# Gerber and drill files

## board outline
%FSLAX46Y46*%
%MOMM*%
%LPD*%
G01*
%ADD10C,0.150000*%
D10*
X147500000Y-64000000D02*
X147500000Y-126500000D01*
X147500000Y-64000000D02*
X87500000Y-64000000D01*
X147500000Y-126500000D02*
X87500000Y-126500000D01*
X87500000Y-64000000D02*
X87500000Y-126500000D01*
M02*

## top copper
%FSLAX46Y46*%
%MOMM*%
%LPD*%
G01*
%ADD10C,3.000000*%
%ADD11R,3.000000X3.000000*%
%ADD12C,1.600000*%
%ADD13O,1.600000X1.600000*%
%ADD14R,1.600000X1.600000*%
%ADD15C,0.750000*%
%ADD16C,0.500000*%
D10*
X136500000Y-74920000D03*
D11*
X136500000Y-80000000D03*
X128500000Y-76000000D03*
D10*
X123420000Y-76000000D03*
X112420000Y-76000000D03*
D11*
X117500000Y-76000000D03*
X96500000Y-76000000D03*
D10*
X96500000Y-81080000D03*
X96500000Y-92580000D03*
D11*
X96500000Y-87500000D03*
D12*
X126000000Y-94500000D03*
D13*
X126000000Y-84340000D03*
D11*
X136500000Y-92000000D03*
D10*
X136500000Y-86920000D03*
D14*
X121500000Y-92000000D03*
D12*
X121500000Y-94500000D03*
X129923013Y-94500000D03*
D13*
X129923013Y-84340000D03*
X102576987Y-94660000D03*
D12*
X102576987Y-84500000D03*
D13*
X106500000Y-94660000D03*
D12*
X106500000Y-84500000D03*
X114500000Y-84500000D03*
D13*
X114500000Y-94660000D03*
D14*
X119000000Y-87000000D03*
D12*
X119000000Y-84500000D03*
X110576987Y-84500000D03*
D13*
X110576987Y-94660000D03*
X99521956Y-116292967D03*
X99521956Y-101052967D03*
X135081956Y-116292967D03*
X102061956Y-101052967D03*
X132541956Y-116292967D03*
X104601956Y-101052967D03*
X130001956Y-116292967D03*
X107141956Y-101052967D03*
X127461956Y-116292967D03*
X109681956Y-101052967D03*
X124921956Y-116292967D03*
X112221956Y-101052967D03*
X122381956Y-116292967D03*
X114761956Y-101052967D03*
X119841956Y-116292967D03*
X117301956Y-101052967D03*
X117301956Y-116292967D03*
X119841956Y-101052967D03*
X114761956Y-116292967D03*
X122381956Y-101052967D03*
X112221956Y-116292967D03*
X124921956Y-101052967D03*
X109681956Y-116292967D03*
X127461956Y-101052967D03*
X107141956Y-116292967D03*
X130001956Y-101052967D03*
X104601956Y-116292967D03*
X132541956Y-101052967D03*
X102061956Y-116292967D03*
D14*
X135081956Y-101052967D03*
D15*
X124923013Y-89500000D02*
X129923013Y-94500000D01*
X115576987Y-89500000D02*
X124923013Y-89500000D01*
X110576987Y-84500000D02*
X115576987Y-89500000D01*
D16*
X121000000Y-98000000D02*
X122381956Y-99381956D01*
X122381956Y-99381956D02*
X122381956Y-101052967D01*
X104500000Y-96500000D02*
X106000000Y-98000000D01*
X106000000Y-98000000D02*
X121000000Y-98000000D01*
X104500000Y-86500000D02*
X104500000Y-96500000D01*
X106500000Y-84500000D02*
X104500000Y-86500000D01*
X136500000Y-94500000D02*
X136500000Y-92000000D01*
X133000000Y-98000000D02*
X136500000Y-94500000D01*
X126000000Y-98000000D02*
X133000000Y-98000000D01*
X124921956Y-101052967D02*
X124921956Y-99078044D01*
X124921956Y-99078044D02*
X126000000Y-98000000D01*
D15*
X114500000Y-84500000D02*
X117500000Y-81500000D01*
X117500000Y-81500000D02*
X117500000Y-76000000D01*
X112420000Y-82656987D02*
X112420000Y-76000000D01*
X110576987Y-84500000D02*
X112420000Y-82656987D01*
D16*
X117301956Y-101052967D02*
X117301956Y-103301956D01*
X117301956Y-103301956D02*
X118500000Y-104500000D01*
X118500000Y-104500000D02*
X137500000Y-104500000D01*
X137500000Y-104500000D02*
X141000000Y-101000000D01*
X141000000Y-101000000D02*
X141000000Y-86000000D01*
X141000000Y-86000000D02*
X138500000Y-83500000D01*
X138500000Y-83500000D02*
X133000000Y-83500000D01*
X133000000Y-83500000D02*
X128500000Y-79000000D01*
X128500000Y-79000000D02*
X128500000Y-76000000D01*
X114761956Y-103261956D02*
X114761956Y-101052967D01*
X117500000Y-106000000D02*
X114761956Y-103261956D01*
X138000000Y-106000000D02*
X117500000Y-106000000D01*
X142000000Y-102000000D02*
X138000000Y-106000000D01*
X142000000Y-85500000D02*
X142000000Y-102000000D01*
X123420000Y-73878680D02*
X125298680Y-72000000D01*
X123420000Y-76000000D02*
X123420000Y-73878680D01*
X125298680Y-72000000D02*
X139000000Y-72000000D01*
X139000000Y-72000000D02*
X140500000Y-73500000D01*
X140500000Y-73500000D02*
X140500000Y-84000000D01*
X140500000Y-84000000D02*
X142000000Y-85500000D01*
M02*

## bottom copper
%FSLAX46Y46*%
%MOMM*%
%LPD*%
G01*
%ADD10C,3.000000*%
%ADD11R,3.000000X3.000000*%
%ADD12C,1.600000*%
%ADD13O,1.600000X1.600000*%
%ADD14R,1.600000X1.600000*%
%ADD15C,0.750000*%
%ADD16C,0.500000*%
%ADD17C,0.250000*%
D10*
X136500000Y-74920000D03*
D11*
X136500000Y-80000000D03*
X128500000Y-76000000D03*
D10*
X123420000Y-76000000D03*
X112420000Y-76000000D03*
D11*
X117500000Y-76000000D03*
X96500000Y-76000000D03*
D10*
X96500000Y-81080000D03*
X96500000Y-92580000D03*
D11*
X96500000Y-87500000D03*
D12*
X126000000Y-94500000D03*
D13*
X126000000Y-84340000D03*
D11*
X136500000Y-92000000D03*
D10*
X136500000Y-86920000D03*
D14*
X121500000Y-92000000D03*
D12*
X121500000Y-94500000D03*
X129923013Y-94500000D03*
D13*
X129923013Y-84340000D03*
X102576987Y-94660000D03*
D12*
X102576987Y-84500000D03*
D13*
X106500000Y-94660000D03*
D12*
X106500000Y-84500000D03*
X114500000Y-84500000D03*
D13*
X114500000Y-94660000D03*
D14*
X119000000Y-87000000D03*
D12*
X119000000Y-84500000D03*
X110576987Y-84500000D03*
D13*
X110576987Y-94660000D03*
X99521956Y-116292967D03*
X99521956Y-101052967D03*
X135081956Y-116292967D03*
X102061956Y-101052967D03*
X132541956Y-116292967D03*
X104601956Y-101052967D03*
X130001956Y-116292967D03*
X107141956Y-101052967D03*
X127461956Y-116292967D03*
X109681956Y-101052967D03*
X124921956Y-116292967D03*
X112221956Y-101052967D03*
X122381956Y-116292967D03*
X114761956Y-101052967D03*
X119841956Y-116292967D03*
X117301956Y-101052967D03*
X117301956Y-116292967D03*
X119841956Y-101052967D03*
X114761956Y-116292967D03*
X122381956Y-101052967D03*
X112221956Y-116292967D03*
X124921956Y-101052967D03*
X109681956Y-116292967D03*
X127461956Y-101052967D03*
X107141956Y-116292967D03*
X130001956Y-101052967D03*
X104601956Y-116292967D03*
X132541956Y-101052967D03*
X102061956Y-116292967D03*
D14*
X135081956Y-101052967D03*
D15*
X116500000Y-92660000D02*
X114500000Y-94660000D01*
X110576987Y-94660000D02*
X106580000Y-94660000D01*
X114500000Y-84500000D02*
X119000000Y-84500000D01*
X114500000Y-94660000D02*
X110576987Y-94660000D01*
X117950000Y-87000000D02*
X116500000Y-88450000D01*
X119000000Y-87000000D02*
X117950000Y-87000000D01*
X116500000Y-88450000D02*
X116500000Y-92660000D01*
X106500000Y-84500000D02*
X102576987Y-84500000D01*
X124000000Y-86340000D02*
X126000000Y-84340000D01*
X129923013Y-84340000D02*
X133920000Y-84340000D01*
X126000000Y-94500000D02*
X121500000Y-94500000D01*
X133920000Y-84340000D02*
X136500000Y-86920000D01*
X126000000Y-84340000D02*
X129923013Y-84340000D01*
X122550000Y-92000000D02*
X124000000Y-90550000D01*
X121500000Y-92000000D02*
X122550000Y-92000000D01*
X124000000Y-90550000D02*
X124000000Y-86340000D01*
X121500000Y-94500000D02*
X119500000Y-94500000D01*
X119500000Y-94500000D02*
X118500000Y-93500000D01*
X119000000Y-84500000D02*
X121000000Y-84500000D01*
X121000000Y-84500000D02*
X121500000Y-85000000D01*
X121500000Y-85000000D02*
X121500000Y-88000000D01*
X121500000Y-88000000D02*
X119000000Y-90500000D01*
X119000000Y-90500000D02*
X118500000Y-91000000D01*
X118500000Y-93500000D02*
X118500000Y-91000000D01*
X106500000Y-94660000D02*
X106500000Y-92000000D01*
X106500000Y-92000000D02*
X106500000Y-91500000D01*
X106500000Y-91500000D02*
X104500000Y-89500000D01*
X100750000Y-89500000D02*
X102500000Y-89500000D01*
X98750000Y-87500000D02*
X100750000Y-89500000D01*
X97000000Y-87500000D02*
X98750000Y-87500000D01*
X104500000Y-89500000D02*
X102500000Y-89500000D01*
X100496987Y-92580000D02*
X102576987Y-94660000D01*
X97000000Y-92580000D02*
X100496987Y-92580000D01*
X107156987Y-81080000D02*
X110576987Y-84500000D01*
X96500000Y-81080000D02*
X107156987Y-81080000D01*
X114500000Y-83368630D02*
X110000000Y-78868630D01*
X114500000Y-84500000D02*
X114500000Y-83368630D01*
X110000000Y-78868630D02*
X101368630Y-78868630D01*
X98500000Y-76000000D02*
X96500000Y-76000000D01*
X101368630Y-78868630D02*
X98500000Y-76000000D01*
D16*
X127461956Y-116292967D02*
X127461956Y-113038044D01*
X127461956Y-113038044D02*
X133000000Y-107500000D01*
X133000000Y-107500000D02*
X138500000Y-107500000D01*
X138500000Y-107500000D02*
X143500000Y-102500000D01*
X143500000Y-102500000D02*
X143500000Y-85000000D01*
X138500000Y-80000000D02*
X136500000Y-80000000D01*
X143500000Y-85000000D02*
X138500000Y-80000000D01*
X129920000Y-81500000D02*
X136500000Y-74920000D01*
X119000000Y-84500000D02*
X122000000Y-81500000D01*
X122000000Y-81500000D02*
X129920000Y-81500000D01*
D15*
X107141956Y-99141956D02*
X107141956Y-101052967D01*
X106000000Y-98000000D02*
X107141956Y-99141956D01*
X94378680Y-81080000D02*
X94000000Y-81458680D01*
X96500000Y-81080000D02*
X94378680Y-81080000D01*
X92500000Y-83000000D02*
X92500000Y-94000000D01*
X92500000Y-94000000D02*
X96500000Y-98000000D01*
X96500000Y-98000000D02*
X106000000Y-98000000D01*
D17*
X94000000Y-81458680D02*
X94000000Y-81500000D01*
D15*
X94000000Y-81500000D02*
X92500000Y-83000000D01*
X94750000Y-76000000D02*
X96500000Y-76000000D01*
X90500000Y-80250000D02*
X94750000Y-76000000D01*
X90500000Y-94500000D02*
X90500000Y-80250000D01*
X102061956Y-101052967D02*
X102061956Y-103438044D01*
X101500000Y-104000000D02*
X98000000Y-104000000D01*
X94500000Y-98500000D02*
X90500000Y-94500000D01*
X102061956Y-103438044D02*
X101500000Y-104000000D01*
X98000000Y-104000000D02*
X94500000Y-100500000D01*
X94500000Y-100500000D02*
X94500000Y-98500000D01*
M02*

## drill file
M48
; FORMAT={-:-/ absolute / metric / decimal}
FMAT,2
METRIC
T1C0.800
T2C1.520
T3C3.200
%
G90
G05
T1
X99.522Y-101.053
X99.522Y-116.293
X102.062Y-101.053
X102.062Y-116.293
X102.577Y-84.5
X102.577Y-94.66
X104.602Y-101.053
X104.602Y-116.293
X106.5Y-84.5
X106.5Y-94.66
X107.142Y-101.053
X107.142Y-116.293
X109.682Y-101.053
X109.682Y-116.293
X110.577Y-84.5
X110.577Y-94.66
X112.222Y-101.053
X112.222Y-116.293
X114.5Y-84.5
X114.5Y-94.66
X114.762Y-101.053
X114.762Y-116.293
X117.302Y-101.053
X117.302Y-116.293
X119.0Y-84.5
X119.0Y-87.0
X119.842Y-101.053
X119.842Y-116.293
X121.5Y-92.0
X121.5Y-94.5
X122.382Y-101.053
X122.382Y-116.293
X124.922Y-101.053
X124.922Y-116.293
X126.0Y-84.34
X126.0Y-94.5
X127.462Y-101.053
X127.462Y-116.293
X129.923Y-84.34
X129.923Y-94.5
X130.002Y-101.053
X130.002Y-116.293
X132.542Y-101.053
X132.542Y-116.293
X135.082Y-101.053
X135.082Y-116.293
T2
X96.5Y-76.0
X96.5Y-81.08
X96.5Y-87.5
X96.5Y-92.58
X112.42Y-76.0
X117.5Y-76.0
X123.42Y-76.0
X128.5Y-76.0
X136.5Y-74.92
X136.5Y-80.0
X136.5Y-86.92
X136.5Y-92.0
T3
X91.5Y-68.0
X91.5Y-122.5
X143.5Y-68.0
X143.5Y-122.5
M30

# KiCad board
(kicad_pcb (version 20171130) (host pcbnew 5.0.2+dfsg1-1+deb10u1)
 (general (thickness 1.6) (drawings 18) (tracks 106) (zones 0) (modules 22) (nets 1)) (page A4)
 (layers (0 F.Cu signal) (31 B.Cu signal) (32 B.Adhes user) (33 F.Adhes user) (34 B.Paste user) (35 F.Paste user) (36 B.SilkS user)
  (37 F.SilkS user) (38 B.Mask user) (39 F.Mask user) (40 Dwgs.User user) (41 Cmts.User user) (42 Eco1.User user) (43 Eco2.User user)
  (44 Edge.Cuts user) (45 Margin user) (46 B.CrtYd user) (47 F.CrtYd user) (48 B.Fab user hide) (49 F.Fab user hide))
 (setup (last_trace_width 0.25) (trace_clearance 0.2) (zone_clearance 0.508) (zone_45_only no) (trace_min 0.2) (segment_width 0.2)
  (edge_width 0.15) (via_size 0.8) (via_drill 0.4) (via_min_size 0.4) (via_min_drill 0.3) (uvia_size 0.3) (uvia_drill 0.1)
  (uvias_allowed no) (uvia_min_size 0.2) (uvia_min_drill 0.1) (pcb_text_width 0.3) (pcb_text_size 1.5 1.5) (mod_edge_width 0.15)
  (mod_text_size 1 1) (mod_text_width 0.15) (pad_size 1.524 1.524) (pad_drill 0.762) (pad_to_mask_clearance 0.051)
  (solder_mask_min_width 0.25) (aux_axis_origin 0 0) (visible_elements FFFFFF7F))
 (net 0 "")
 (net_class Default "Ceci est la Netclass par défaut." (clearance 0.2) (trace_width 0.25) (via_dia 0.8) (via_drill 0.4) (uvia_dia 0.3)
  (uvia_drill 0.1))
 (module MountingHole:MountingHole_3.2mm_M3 (layer F.Cu) (at 91.5 68)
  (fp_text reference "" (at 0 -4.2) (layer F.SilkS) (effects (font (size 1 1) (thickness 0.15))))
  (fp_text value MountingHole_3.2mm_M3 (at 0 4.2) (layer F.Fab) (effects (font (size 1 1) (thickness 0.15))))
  (pad 1 np_thru_hole circle (at 0 0) (size 3.2 3.2) (drill 3.2) (layers *.Cu *.Mask)))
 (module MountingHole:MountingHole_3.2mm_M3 (layer F.Cu) (at 143.5 68)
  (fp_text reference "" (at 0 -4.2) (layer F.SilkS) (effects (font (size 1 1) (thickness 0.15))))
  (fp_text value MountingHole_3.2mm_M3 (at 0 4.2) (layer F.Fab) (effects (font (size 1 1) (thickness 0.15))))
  (pad 1 np_thru_hole circle (at 0 0) (size 3.2 3.2) (drill 3.2) (layers *.Cu *.Mask)))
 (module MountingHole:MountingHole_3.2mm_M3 (layer F.Cu) (at 143.5 122.5)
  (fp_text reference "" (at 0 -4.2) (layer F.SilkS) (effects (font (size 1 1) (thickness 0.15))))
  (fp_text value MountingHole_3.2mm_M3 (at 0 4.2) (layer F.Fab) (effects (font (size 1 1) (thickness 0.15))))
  (pad 1 np_thru_hole circle (at 0 0) (size 3.2 3.2) (drill 3.2) (layers *.Cu *.Mask)))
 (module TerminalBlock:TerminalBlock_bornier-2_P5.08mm (layer F.Cu) (at 136.5 80 90)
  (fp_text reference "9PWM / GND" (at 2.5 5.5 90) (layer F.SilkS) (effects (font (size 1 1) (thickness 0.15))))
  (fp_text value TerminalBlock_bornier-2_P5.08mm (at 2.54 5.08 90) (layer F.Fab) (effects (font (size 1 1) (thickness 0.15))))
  (pad 2 thru_hole circle (at 5.08 0 90) (size 3 3) (drill 1.52) (layers *.Cu *.Mask))
  (pad 1 thru_hole rect (at 0 0 90) (size 3 3) (drill 1.52) (layers *.Cu *.Mask)))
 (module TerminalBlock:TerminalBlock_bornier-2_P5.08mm (layer F.Cu) (at 128.5 76 180)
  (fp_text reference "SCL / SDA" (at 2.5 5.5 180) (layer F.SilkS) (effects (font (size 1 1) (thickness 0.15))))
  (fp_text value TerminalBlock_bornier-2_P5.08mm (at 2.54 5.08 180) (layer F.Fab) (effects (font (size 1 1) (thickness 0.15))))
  (pad 1 thru_hole rect (at 0 0 180) (size 3 3) (drill 1.52) (layers *.Cu *.Mask))
  (pad 2 thru_hole circle (at 5.08 0 180) (size 3 3) (drill 1.52) (layers *.Cu *.Mask)))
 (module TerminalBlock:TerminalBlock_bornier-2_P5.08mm (layer F.Cu) (at 117.5 76 180)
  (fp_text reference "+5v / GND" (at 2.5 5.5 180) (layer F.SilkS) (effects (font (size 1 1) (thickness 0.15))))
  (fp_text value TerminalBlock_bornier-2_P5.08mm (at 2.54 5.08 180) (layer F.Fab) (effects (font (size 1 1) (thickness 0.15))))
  (pad 2 thru_hole circle (at 5.08 0 180) (size 3 3) (drill 1.52) (layers *.Cu *.Mask))
  (pad 1 thru_hole rect (at 0 0 180) (size 3 3) (drill 1.52) (layers *.Cu *.Mask)))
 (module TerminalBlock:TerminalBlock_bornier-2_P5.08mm (layer F.Cu) (at 96.5 76 270)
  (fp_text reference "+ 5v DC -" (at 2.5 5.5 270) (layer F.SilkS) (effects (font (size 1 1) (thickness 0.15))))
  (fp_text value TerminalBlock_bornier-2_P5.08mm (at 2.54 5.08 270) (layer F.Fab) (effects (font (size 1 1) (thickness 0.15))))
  (pad 1 thru_hole rect (at 0 0 270) (size 3 3) (drill 1.52) (layers *.Cu *.Mask))
  (pad 2 thru_hole circle (at 5.08 0 270) (size 3 3) (drill 1.52) (layers *.Cu *.Mask)))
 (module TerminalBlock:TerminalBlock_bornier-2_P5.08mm (layer F.Cu) (at 96.5 87.5 270)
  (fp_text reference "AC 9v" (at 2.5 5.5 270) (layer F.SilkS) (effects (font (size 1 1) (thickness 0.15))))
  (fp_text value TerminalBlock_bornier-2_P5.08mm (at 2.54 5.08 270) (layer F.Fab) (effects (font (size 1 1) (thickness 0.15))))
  (pad 2 thru_hole circle (at 5.08 0 270) (size 3 3) (drill 1.52) (layers *.Cu *.Mask))
  (pad 1 thru_hole rect (at 0 0 270) (size 3 3) (drill 1.52) (layers *.Cu *.Mask)))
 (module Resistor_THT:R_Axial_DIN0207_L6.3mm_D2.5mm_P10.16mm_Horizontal (layer F.Cu) (at 126 94.5 90)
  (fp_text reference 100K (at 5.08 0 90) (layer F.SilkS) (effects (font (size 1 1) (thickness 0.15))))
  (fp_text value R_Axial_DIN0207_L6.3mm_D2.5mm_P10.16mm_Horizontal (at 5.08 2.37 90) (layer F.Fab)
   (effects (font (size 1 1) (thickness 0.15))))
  (pad 1 thru_hole circle (at 0 0 90) (size 1.6 1.6) (drill 0.8) (layers *.Cu *.Mask))
  (pad 2 thru_hole oval (at 10.16 0 90) (size 1.6 1.6) (drill 0.8) (layers *.Cu *.Mask)))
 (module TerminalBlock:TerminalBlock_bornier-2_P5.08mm (layer F.Cu) (at 136.5 92 90)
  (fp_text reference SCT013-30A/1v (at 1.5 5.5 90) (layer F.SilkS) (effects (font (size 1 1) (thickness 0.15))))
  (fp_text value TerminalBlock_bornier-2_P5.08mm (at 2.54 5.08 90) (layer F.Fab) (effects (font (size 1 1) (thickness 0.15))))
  (pad 1 thru_hole rect (at 0 0 90) (size 3 3) (drill 1.52) (layers *.Cu *.Mask))
  (pad 2 thru_hole circle (at 5.08 0 90) (size 3 3) (drill 1.52) (layers *.Cu *.Mask)))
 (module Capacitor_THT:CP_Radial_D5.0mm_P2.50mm (layer F.Cu) (at 121.5 92 270)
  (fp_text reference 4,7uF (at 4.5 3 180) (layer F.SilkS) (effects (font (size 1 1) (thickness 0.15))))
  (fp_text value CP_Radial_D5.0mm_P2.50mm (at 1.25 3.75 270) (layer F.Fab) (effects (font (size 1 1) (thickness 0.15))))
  (pad 1 thru_hole rect (at 0 0 270) (size 1.6 1.6) (drill 0.8) (layers *.Cu *.Mask))
  (pad 2 thru_hole circle (at 2.5 0 270) (size 1.6 1.6) (drill 0.8) (layers *.Cu *.Mask)))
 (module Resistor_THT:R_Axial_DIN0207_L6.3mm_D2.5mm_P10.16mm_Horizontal (layer F.Cu) (at 129.923013 94.5 90)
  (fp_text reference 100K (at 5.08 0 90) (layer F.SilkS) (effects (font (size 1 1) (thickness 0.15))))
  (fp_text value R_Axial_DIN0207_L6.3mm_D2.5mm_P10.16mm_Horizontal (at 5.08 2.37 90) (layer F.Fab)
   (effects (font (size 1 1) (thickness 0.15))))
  (pad 1 thru_hole circle (at 0 0 90) (size 1.6 1.6) (drill 0.8) (layers *.Cu *.Mask))
  (pad 2 thru_hole oval (at 10.16 0 90) (size 1.6 1.6) (drill 0.8) (layers *.Cu *.Mask)))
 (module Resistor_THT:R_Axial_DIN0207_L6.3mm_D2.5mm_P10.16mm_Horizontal (layer F.Cu) (at 102.576987 84.5 270)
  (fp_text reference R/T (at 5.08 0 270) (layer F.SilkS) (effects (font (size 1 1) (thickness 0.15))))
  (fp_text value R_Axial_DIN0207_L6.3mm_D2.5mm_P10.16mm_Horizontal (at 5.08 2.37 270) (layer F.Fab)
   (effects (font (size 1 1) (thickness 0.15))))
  (pad 2 thru_hole oval (at 10.16 0 270) (size 1.6 1.6) (drill 0.8) (layers *.Cu *.Mask))
  (pad 1 thru_hole circle (at 0 0 270) (size 1.6 1.6) (drill 0.8) (layers *.Cu *.Mask)))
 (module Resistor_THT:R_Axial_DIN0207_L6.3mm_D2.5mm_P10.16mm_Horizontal (layer F.Cu) (at 106.5 84.5 270)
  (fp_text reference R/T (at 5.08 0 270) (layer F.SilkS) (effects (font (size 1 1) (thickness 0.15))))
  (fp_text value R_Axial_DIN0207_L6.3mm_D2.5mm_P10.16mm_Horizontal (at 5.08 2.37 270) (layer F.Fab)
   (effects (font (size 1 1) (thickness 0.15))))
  (pad 2 thru_hole oval (at 10.16 0 270) (size 1.6 1.6) (drill 0.8) (layers *.Cu *.Mask))
  (pad 1 thru_hole circle (at 0 0 270) (size 1.6 1.6) (drill 0.8) (layers *.Cu *.Mask)))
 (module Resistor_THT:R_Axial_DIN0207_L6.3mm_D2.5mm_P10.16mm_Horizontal (layer F.Cu) (at 114.5 84.5 270)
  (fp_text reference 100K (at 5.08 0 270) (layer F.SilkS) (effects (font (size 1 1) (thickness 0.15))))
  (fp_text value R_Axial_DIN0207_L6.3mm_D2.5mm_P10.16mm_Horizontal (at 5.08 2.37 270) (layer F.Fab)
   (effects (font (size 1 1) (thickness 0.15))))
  (pad 1 thru_hole circle (at 0 0 270) (size 1.6 1.6) (drill 0.8) (layers *.Cu *.Mask))
  (pad 2 thru_hole oval (at 10.16 0 270) (size 1.6 1.6) (drill 0.8) (layers *.Cu *.Mask)))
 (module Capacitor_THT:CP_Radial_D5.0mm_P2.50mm (layer F.Cu) (at 119 87 90)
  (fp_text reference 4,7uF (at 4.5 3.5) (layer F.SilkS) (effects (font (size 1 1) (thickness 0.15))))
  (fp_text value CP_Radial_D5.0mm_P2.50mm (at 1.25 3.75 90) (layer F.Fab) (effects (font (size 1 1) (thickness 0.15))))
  (pad 1 thru_hole rect (at 0 0 90) (size 1.6 1.6) (drill 0.8) (layers *.Cu *.Mask))
  (pad 2 thru_hole circle (at 2.5 0 90) (size 1.6 1.6) (drill 0.8) (layers *.Cu *.Mask)))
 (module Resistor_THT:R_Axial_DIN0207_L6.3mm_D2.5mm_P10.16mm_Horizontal (layer F.Cu) (at 110.576987 84.5 270)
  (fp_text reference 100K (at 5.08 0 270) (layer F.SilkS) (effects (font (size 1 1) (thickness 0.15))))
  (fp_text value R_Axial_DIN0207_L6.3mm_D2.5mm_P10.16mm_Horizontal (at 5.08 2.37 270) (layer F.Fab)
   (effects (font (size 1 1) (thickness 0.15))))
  (pad 1 thru_hole circle (at 0 0 270) (size 1.6 1.6) (drill 0.8) (layers *.Cu *.Mask))
  (pad 2 thru_hole oval (at 10.16 0 270) (size 1.6 1.6) (drill 0.8) (layers *.Cu *.Mask)))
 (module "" (layer F.Cu) (at 72 144.5)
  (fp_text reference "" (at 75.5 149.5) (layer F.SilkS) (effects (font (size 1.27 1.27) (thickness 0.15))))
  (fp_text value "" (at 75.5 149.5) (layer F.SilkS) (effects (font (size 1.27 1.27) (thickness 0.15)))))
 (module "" (layer F.Cu) (at 45.5 145)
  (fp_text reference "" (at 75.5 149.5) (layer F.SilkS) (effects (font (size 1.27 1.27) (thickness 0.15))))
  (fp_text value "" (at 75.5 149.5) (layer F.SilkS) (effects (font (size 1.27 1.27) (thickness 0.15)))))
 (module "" (layer F.Cu) (at 80 110.5)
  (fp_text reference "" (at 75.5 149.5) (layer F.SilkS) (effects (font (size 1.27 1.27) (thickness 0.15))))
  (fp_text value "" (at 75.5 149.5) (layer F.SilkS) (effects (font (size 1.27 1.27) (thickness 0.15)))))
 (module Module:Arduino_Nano (layer F.Cu) (at 135.081956 101.052967 270)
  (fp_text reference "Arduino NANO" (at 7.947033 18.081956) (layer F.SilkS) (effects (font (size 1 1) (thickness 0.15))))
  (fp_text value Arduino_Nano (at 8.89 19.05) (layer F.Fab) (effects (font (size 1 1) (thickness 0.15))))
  (pad 16 thru_hole oval (at 15.24 35.56 270) (size 1.6 1.6) (drill 0.8) (layers *.Cu *.Mask))
  (pad 15 thru_hole oval (at 0 35.56 270) (size 1.6 1.6) (drill 0.8) (layers *.Cu *.Mask))
  (pad 30 thru_hole oval (at 15.24 0 270) (size 1.6 1.6) (drill 0.8) (layers *.Cu *.Mask))
  (pad 14 thru_hole oval (at 0 33.02 270) (size 1.6 1.6) (drill 0.8) (layers *.Cu *.Mask))
  (pad 29 thru_hole oval (at 15.24 2.54 270) (size 1.6 1.6) (drill 0.8) (layers *.Cu *.Mask))
  (pad 13 thru_hole oval (at 0 30.48 270) (size 1.6 1.6) (drill 0.8) (layers *.Cu *.Mask))
  (pad 28 thru_hole oval (at 15.24 5.08 270) (size 1.6 1.6) (drill 0.8) (layers *.Cu *.Mask))
  (pad 12 thru_hole oval (at 0 27.94 270) (size 1.6 1.6) (drill 0.8) (layers *.Cu *.Mask))
  (pad 27 thru_hole oval (at 15.24 7.62 270) (size 1.6 1.6) (drill 0.8) (layers *.Cu *.Mask))
  (pad 11 thru_hole oval (at 0 25.4 270) (size 1.6 1.6) (drill 0.8) (layers *.Cu *.Mask))
  (pad 26 thru_hole oval (at 15.24 10.16 270) (size 1.6 1.6) (drill 0.8) (layers *.Cu *.Mask))
  (pad 10 thru_hole oval (at 0 22.86 270) (size 1.6 1.6) (drill 0.8) (layers *.Cu *.Mask))
  (pad 25 thru_hole oval (at 15.24 12.7 270) (size 1.6 1.6) (drill 0.8) (layers *.Cu *.Mask))
  (pad 9 thru_hole oval (at 0 20.32 270) (size 1.6 1.6) (drill 0.8) (layers *.Cu *.Mask))
  (pad 24 thru_hole oval (at 15.24 15.24 270) (size 1.6 1.6) (drill 0.8) (layers *.Cu *.Mask))
  (pad 8 thru_hole oval (at 0 17.78 270) (size 1.6 1.6) (drill 0.8) (layers *.Cu *.Mask))
  (pad 23 thru_hole oval (at 15.24 17.78 270) (size 1.6 1.6) (drill 0.8) (layers *.Cu *.Mask))
  (pad 7 thru_hole oval (at 0 15.24 270) (size 1.6 1.6) (drill 0.8) (layers *.Cu *.Mask))
  (pad 22 thru_hole oval (at 15.24 20.32 270) (size 1.6 1.6) (drill 0.8) (layers *.Cu *.Mask))
  (pad 6 thru_hole oval (at 0 12.7 270) (size 1.6 1.6) (drill 0.8) (layers *.Cu *.Mask))
  (pad 21 thru_hole oval (at 15.24 22.86 270) (size 1.6 1.6) (drill 0.8) (layers *.Cu *.Mask))
  (pad 5 thru_hole oval (at 0 10.16 270) (size 1.6 1.6) (drill 0.8) (layers *.Cu *.Mask))
  (pad 20 thru_hole oval (at 15.24 25.4 270) (size 1.6 1.6) (drill 0.8) (layers *.Cu *.Mask))
  (pad 4 thru_hole oval (at 0 7.62 270) (size 1.6 1.6) (drill 0.8) (layers *.Cu *.Mask))
  (pad 19 thru_hole oval (at 15.24 27.94 270) (size 1.6 1.6) (drill 0.8) (layers *.Cu *.Mask))
  (pad 3 thru_hole oval (at 0 5.08 270) (size 1.6 1.6) (drill 0.8) (layers *.Cu *.Mask))
  (pad 18 thru_hole oval (at 15.24 30.48 270) (size 1.6 1.6) (drill 0.8) (layers *.Cu *.Mask))
  (pad 2 thru_hole oval (at 0 2.54 270) (size 1.6 1.6) (drill 0.8) (layers *.Cu *.Mask))
  (pad 17 thru_hole oval (at 15.24 33.02 270) (size 1.6 1.6) (drill 0.8) (layers *.Cu *.Mask))
  (pad 1 thru_hole rect (at 0 0 270) (size 1.6 1.6) (drill 0.8) (layers *.Cu *.Mask)))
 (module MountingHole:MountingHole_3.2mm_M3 (layer F.Cu) (at 91.5 122.5)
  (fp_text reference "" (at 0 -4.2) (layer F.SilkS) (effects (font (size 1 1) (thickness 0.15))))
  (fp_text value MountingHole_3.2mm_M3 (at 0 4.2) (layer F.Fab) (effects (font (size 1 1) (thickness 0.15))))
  (pad 1 np_thru_hole circle (at 0 0) (size 3.2 3.2) (drill 3.2) (layers *.Cu *.Mask)))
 (gr_line (start 147.5 64) (end 147.5 126.5) (layer Edge.Cuts) (width 0.15))
 (gr_line (start 147.5 64) (end 87.5 64) (layer Edge.Cuts) (width 0.15))
 (gr_line (start 147.5 126.5) (end 87.5 126.5) (layer Edge.Cuts) (width 0.15))
 (gr_line (start 87.5 64) (end 87.5 126.5) (layer Edge.Cuts) (width 0.15))
 (segment (start 116.5 92.66) (end 114.5 94.66) (width 0.75) (layer B.Cu) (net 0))
 (segment (start 110.576987 94.66) (end 106.58 94.66) (width 0.75) (layer B.Cu) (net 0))
 (segment (start 114.5 84.5) (end 119 84.5) (width 0.75) (layer B.Cu) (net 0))
 (segment (start 114.5 94.66) (end 110.576987 94.66) (width 0.75) (layer B.Cu) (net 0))
 (segment (start 117.95 87) (end 116.5 88.45) (width 0.75) (layer B.Cu) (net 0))
 (segment (start 119 87) (end 117.95 87) (width 0.75) (layer B.Cu) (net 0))
 (segment (start 116.5 88.45) (end 116.5 92.66) (width 0.75) (layer B.Cu) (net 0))
 (segment (start 106.5 84.5) (end 102.576987 84.5) (width 0.75) (layer B.Cu) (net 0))
 (segment (start 124 86.34) (end 126 84.34) (width 0.75) (layer B.Cu) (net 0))
 (segment (start 129.923013 84.34) (end 133.92 84.34) (width 0.75) (layer B.Cu) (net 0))
 (segment (start 126 94.5) (end 121.5 94.5) (width 0.75) (layer B.Cu) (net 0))
 (segment (start 133.92 84.34) (end 136.5 86.92) (width 0.75) (layer B.Cu) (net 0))
 (segment (start 126 84.34) (end 129.923013 84.34) (width 0.75) (layer B.Cu) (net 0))
 (segment (start 122.55 92) (end 124 90.55) (width 0.75) (layer B.Cu) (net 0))
 (segment (start 121.5 92) (end 122.55 92) (width 0.75) (layer B.Cu) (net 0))
 (segment (start 124 90.55) (end 124 86.34) (width 0.75) (layer B.Cu) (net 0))
 (segment (start 121.5 94.5) (end 119.5 94.5) (width 0.75) (layer B.Cu) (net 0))
 (segment (start 119.5 94.5) (end 118.5 93.5) (width 0.75) (layer B.Cu) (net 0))
 (segment (start 119 84.5) (end 121 84.5) (width 0.75) (layer B.Cu) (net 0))
 (segment (start 121 84.5) (end 121.5 85) (width 0.75) (layer B.Cu) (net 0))
 (segment (start 121.5 85) (end 121.5 88) (width 0.75) (layer B.Cu) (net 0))
 (segment (start 121.5 88) (end 119 90.5) (width 0.75) (layer B.Cu) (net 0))
 (segment (start 119 90.5) (end 118.5 91) (width 0.75) (layer B.Cu) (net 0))
 (segment (start 118.5 93.5) (end 118.5 91) (width 0.75) (layer B.Cu) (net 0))
 (segment (start 124.923013 89.5) (end 129.923013 94.5) (width 0.75) (layer F.Cu) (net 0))
 (segment (start 115.576987 89.5) (end 124.923013 89.5) (width 0.75) (layer F.Cu) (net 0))
 (segment (start 110.576987 84.5) (end 115.576987 89.5) (width 0.75) (layer F.Cu) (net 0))
 (segment (start 106.5 94.66) (end 106.5 92) (width 0.75) (layer B.Cu) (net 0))
 (segment (start 106.5 92) (end 106.5 91.5) (width 0.75) (layer B.Cu) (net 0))
 (segment (start 106.5 91.5) (end 104.5 89.5) (width 0.75) (layer B.Cu) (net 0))
 (segment (start 100.75 89.5) (end 102.5 89.5) (width 0.75) (layer B.Cu) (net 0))
 (segment (start 98.75 87.5) (end 100.75 89.5) (width 0.75) (layer B.Cu) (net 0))
 (segment (start 97 87.5) (end 98.75 87.5) (width 0.75) (layer B.Cu) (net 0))
 (segment (start 104.5 89.5) (end 102.5 89.5) (width 0.75) (layer B.Cu) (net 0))
 (segment (start 100.496987 92.58) (end 102.576987 94.66) (width 0.75) (layer B.Cu) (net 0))
 (segment (start 97 92.58) (end 100.496987 92.58) (width 0.75) (layer B.Cu) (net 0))
 (segment (start 121 98) (end 122.381956 99.381956) (width 0.5) (layer F.Cu) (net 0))
 (segment (start 122.381956 99.381956) (end 122.381956 101.052967) (width 0.5) (layer F.Cu) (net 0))
 (segment (start 104.5 96.5) (end 106 98) (width 0.5) (layer F.Cu) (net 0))
 (segment (start 106 98) (end 121 98) (width 0.5) (layer F.Cu) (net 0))
 (segment (start 104.5 86.5) (end 104.5 96.5) (width 0.5) (layer F.Cu) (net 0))
 (segment (start 106.5 84.5) (end 104.5 86.5) (width 0.5) (layer F.Cu) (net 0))
 (segment (start 136.5 94.5) (end 136.5 92) (width 0.5) (layer F.Cu) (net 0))
 (segment (start 133 98) (end 136.5 94.5) (width 0.5) (layer F.Cu) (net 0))
 (segment (start 126 98) (end 133 98) (width 0.5) (layer F.Cu) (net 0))
 (segment (start 124.921956 101.052967) (end 124.921956 99.078044) (width 0.5) (layer F.Cu) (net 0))
 (segment (start 124.921956 99.078044) (end 126 98) (width 0.5) (layer F.Cu) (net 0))
 (segment (start 107.156987 81.08) (end 110.576987 84.5) (width 0.75) (layer B.Cu) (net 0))
 (segment (start 96.5 81.08) (end 107.156987 81.08) (width 0.75) (layer B.Cu) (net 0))
 (segment (start 114.5 83.36863) (end 110 78.86863) (width 0.75) (layer B.Cu) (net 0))
 (segment (start 114.5 84.5) (end 114.5 83.36863) (width 0.75) (layer B.Cu) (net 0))
 (segment (start 110 78.86863) (end 101.36863 78.86863) (width 0.75) (layer B.Cu) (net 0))
 (segment (start 98.5 76) (end 96.5 76) (width 0.75) (layer B.Cu) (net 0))
 (segment (start 101.36863 78.86863) (end 98.5 76) (width 0.75) (layer B.Cu) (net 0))
 (segment (start 114.5 84.5) (end 117.5 81.5) (width 0.75) (layer F.Cu) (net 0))
 (segment (start 117.5 81.5) (end 117.5 76) (width 0.75) (layer F.Cu) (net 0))
 (segment (start 112.42 82.656987) (end 112.42 76) (width 0.75) (layer F.Cu) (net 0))
 (segment (start 110.576987 84.5) (end 112.42 82.656987) (width 0.75) (layer F.Cu) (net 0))
 (segment (start 117.301956 101.052967) (end 117.301956 103.301956) (width 0.5) (layer F.Cu) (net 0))
 (segment (start 117.301956 103.301956) (end 118.5 104.5) (width 0.5) (layer F.Cu) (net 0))
 (segment (start 118.5 104.5) (end 137.5 104.5) (width 0.5) (layer F.Cu) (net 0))
 (segment (start 137.5 104.5) (end 141 101) (width 0.5) (layer F.Cu) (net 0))
 (segment (start 141 101) (end 141 86) (width 0.5) (layer F.Cu) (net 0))
 (segment (start 141 86) (end 138.5 83.5) (width 0.5) (layer F.Cu) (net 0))
 (segment (start 138.5 83.5) (end 133 83.5) (width 0.5) (layer F.Cu) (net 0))
 (segment (start 133 83.5) (end 128.5 79) (width 0.5) (layer F.Cu) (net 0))
 (segment (start 128.5 79) (end 128.5 76) (width 0.5) (layer F.Cu) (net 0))
 (segment (start 114.761956 103.261956) (end 114.761956 101.052967) (width 0.5) (layer F.Cu) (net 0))
 (segment (start 117.5 106) (end 114.761956 103.261956) (width 0.5) (layer F.Cu) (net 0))
 (segment (start 138 106) (end 117.5 106) (width 0.5) (layer F.Cu) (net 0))
 (segment (start 142 102) (end 138 106) (width 0.5) (layer F.Cu) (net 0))
 (segment (start 142 85.5) (end 142 102) (width 0.5) (layer F.Cu) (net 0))
 (segment (start 123.42 73.87868) (end 125.29868 72) (width 0.5) (layer F.Cu) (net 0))
 (segment (start 123.42 76) (end 123.42 73.87868) (width 0.5) (layer F.Cu) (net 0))
 (segment (start 125.29868 72) (end 139 72) (width 0.5) (layer F.Cu) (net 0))
 (segment (start 139 72) (end 140.5 73.5) (width 0.5) (layer F.Cu) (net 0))
 (segment (start 140.5 73.5) (end 140.5 84) (width 0.5) (layer F.Cu) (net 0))
 (segment (start 140.5 84) (end 142 85.5) (width 0.5) (layer F.Cu) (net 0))
 (segment (start 127.461956 116.292967) (end 127.461956 113.038044) (width 0.5) (layer B.Cu) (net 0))
 (segment (start 127.461956 113.038044) (end 133 107.5) (width 0.5) (layer B.Cu) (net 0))
 (segment (start 133 107.5) (end 138.5 107.5) (width 0.5) (layer B.Cu) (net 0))
 (segment (start 138.5 107.5) (end 143.5 102.5) (width 0.5) (layer B.Cu) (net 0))
 (segment (start 143.5 102.5) (end 143.5 85) (width 0.5) (layer B.Cu) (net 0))
 (segment (start 138.5 80) (end 136.5 80) (width 0.5) (layer B.Cu) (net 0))
 (segment (start 143.5 85) (end 138.5 80) (width 0.5) (layer B.Cu) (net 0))
 (segment (start 129.92 81.5) (end 136.5 74.92) (width 0.5) (layer B.Cu) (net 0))
 (segment (start 119 84.5) (end 122 81.5) (width 0.5) (layer B.Cu) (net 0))
 (segment (start 122 81.5) (end 129.92 81.5) (width 0.5) (layer B.Cu) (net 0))
 (segment (start 107.141956 99.141956) (end 107.141956 101.052967) (width 0.75) (layer B.Cu) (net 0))
 (segment (start 106 98) (end 107.141956 99.141956) (width 0.75) (layer B.Cu) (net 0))
 (segment (start 94.37868 81.08) (end 94 81.45868) (width 0.75) (layer B.Cu) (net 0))
 (segment (start 96.5 81.08) (end 94.37868 81.08) (width 0.75) (layer B.Cu) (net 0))
 (segment (start 92.5 83) (end 92.5 94) (width 0.75) (layer B.Cu) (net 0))
 (segment (start 92.5 94) (end 96.5 98) (width 0.75) (layer B.Cu) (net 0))
 (segment (start 96.5 98) (end 106 98) (width 0.75) (layer B.Cu) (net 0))
 (segment (start 94 81.45868) (end 94 81.5) (width 0.25) (layer B.Cu) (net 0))
 (segment (start 94 81.5) (end 92.5 83) (width 0.75) (layer B.Cu) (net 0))
 (segment (start 94.75 76) (end 96.5 76) (width 0.75) (layer B.Cu) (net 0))
 (segment (start 90.5 80.25) (end 94.75 76) (width 0.75) (layer B.Cu) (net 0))
 (segment (start 90.5 94.5) (end 90.5 80.25) (width 0.75) (layer B.Cu) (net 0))
 (segment (start 102.061956 101.052967) (end 102.061956 103.438044) (width 0.75) (layer B.Cu) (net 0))
 (segment (start 101.5 104) (end 98 104) (width 0.75) (layer B.Cu) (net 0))
 (segment (start 94.5 98.5) (end 90.5 94.5) (width 0.75) (layer B.Cu) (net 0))
 (segment (start 102.061956 103.438044) (end 101.5 104) (width 0.75) (layer B.Cu) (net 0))
 (segment (start 98 104) (end 94.5 100.5) (width 0.75) (layer B.Cu) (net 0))
 (segment (start 94.5 100.5) (end 94.5 98.5) (width 0.75) (layer B.Cu) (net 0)))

